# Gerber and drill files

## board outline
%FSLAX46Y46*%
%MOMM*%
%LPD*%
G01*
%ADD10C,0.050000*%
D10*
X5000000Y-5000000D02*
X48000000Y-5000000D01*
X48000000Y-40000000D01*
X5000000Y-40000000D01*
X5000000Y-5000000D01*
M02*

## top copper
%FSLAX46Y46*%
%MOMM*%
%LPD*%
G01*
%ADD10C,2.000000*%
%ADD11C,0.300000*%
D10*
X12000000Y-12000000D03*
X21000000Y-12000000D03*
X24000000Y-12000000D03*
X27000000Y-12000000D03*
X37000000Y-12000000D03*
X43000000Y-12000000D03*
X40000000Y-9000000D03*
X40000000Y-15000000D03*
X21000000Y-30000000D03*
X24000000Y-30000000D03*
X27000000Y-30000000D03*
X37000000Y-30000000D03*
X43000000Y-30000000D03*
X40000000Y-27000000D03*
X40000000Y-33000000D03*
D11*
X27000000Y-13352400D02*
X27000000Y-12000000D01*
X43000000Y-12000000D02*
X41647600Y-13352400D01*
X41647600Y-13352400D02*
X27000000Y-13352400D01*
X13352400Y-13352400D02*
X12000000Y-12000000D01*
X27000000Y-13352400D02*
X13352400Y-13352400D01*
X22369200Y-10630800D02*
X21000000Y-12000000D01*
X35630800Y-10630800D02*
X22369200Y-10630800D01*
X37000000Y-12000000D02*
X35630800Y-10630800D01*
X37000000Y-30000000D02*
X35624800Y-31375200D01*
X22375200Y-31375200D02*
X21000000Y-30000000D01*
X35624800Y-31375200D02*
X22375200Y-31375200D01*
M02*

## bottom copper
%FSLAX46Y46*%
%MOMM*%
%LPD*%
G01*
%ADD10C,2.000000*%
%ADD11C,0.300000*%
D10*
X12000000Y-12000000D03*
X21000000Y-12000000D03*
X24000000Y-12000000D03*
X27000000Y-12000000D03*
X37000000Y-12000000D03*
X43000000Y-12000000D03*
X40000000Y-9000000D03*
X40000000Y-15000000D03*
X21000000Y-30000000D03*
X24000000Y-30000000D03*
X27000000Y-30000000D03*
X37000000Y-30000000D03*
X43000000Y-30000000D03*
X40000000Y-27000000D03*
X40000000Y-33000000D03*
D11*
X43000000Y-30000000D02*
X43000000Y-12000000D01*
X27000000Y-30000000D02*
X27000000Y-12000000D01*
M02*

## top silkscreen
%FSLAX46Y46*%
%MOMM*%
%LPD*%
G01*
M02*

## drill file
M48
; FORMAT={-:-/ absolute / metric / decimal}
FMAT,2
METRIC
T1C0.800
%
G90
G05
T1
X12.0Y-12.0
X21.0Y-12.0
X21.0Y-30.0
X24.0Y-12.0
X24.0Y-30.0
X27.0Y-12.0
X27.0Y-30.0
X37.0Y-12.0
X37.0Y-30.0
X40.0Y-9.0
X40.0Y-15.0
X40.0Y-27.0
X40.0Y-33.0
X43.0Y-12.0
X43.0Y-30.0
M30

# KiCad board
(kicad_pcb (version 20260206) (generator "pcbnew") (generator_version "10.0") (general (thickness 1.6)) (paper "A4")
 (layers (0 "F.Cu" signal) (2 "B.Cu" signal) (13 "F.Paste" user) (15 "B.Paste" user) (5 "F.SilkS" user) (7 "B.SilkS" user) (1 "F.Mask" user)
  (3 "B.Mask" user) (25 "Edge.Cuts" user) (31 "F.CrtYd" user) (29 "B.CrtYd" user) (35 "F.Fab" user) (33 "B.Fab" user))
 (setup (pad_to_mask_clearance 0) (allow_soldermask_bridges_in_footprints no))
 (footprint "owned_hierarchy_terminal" (layer "F.Cu") (at 12 12)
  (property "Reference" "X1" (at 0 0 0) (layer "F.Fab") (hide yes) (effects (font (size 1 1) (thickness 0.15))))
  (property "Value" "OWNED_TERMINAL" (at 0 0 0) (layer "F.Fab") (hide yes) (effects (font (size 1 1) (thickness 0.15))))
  (pad "1" thru_hole circle (at 0 0) (size 2 2) (drill 0.8) (layers "*.Cu" "*.Mask") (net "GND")))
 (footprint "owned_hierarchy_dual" (layer "F.Cu") (at 24 12)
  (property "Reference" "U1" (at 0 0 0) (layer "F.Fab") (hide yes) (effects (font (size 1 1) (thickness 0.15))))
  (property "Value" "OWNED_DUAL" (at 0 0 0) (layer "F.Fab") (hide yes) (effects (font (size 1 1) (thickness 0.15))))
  (pad "1" thru_hole circle (at -3 0) (size 2 2) (drill 0.8) (layers "*.Cu" "*.Mask") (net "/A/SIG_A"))
  (pad "2" thru_hole circle (at 0 0) (size 2 2) (drill 0.8) (layers "*.Cu" "*.Mask") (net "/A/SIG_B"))
  (pad "3" thru_hole circle (at 3 0) (size 2 2) (drill 0.8) (layers "*.Cu" "*.Mask") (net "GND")))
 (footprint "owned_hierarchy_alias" (layer "F.Cu") (at 40 12)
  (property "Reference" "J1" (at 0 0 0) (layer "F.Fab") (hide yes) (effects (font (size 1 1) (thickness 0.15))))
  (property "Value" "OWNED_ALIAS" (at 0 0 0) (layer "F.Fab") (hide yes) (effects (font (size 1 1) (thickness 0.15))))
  (pad "R" thru_hole circle (at -3 0) (size 2 2) (drill 0.8) (layers "*.Cu" "*.Mask") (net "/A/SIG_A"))
  (pad "T" thru_hole circle (at 3 0) (size 2 2) (drill 0.8) (layers "*.Cu" "*.Mask") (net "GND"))
  (pad "MP" thru_hole circle (at 0 -3) (size 2 2) (drill 0.8) (layers "*.Cu" "*.Mask"))
  (pad "MP" thru_hole circle (at 0 3) (size 2 2) (drill 0.8) (layers "*.Cu" "*.Mask")))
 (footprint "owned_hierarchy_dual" (layer "F.Cu") (at 24 30)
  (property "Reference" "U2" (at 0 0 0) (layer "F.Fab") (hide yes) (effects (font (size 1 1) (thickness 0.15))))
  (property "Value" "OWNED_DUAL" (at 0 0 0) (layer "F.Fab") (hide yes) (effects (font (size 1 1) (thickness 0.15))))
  (pad "1" thru_hole circle (at -3 0) (size 2 2) (drill 0.8) (layers "*.Cu" "*.Mask") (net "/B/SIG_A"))
  (pad "2" thru_hole circle (at 0 0) (size 2 2) (drill 0.8) (layers "*.Cu" "*.Mask") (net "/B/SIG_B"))
  (pad "3" thru_hole circle (at 3 0) (size 2 2) (drill 0.8) (layers "*.Cu" "*.Mask") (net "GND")))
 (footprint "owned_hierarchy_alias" (layer "F.Cu") (at 40 30)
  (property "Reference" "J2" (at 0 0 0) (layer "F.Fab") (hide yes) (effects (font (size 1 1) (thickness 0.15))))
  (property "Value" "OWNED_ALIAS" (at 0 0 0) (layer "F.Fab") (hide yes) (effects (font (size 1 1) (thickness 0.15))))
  (pad "R" thru_hole circle (at -3 0) (size 2 2) (drill 0.8) (layers "*.Cu" "*.Mask") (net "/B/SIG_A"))
  (pad "T" thru_hole circle (at 3 0) (size 2 2) (drill 0.8) (layers "*.Cu" "*.Mask") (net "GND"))
  (pad "MP" thru_hole circle (at 0 -3) (size 2 2) (drill 0.8) (layers "*.Cu" "*.Mask"))
  (pad "MP" thru_hole circle (at 0 3) (size 2 2) (drill 0.8) (layers "*.Cu" "*.Mask")))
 (gr_rect (start 5 5) (end 48 40) (stroke (width 0.05) (type default)) (fill none) (layer "Edge.Cuts"))
 (segment (start 27 13.3524) (end 27 12) (width 0.3) (layer "F.Cu") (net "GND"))
 (segment (start 43 12) (end 41.6476 13.3524) (width 0.3) (layer "F.Cu") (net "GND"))
 (segment (start 41.6476 13.3524) (end 27 13.3524) (width 0.3) (layer "F.Cu") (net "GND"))
 (segment (start 13.3524 13.3524) (end 12 12) (width 0.3) (layer "F.Cu") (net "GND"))
 (segment (start 27 13.3524) (end 13.3524 13.3524) (width 0.3) (layer "F.Cu") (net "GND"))
 (segment (start 43 30) (end 43 12) (width 0.3) (layer "B.Cu") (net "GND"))
 (segment (start 27 30) (end 27 12) (width 0.3) (layer "B.Cu") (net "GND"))
 (segment (start 22.3692 10.6308) (end 21 12) (width 0.3) (layer "F.Cu") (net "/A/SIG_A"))
 (segment (start 35.6308 10.6308) (end 22.3692 10.6308) (width 0.3) (layer "F.Cu") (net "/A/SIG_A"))
 (segment (start 37 12) (end 35.6308 10.6308) (width 0.3) (layer "F.Cu") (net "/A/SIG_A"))
 (segment (start 37 30) (end 35.6248 31.3752) (width 0.3) (layer "F.Cu") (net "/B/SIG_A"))
 (segment (start 22.3752 31.3752) (end 21 30) (width 0.3) (layer "F.Cu") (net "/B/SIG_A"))
 (segment (start 35.6248 31.3752) (end 22.3752 31.3752) (width 0.3) (layer "F.Cu") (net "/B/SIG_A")))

